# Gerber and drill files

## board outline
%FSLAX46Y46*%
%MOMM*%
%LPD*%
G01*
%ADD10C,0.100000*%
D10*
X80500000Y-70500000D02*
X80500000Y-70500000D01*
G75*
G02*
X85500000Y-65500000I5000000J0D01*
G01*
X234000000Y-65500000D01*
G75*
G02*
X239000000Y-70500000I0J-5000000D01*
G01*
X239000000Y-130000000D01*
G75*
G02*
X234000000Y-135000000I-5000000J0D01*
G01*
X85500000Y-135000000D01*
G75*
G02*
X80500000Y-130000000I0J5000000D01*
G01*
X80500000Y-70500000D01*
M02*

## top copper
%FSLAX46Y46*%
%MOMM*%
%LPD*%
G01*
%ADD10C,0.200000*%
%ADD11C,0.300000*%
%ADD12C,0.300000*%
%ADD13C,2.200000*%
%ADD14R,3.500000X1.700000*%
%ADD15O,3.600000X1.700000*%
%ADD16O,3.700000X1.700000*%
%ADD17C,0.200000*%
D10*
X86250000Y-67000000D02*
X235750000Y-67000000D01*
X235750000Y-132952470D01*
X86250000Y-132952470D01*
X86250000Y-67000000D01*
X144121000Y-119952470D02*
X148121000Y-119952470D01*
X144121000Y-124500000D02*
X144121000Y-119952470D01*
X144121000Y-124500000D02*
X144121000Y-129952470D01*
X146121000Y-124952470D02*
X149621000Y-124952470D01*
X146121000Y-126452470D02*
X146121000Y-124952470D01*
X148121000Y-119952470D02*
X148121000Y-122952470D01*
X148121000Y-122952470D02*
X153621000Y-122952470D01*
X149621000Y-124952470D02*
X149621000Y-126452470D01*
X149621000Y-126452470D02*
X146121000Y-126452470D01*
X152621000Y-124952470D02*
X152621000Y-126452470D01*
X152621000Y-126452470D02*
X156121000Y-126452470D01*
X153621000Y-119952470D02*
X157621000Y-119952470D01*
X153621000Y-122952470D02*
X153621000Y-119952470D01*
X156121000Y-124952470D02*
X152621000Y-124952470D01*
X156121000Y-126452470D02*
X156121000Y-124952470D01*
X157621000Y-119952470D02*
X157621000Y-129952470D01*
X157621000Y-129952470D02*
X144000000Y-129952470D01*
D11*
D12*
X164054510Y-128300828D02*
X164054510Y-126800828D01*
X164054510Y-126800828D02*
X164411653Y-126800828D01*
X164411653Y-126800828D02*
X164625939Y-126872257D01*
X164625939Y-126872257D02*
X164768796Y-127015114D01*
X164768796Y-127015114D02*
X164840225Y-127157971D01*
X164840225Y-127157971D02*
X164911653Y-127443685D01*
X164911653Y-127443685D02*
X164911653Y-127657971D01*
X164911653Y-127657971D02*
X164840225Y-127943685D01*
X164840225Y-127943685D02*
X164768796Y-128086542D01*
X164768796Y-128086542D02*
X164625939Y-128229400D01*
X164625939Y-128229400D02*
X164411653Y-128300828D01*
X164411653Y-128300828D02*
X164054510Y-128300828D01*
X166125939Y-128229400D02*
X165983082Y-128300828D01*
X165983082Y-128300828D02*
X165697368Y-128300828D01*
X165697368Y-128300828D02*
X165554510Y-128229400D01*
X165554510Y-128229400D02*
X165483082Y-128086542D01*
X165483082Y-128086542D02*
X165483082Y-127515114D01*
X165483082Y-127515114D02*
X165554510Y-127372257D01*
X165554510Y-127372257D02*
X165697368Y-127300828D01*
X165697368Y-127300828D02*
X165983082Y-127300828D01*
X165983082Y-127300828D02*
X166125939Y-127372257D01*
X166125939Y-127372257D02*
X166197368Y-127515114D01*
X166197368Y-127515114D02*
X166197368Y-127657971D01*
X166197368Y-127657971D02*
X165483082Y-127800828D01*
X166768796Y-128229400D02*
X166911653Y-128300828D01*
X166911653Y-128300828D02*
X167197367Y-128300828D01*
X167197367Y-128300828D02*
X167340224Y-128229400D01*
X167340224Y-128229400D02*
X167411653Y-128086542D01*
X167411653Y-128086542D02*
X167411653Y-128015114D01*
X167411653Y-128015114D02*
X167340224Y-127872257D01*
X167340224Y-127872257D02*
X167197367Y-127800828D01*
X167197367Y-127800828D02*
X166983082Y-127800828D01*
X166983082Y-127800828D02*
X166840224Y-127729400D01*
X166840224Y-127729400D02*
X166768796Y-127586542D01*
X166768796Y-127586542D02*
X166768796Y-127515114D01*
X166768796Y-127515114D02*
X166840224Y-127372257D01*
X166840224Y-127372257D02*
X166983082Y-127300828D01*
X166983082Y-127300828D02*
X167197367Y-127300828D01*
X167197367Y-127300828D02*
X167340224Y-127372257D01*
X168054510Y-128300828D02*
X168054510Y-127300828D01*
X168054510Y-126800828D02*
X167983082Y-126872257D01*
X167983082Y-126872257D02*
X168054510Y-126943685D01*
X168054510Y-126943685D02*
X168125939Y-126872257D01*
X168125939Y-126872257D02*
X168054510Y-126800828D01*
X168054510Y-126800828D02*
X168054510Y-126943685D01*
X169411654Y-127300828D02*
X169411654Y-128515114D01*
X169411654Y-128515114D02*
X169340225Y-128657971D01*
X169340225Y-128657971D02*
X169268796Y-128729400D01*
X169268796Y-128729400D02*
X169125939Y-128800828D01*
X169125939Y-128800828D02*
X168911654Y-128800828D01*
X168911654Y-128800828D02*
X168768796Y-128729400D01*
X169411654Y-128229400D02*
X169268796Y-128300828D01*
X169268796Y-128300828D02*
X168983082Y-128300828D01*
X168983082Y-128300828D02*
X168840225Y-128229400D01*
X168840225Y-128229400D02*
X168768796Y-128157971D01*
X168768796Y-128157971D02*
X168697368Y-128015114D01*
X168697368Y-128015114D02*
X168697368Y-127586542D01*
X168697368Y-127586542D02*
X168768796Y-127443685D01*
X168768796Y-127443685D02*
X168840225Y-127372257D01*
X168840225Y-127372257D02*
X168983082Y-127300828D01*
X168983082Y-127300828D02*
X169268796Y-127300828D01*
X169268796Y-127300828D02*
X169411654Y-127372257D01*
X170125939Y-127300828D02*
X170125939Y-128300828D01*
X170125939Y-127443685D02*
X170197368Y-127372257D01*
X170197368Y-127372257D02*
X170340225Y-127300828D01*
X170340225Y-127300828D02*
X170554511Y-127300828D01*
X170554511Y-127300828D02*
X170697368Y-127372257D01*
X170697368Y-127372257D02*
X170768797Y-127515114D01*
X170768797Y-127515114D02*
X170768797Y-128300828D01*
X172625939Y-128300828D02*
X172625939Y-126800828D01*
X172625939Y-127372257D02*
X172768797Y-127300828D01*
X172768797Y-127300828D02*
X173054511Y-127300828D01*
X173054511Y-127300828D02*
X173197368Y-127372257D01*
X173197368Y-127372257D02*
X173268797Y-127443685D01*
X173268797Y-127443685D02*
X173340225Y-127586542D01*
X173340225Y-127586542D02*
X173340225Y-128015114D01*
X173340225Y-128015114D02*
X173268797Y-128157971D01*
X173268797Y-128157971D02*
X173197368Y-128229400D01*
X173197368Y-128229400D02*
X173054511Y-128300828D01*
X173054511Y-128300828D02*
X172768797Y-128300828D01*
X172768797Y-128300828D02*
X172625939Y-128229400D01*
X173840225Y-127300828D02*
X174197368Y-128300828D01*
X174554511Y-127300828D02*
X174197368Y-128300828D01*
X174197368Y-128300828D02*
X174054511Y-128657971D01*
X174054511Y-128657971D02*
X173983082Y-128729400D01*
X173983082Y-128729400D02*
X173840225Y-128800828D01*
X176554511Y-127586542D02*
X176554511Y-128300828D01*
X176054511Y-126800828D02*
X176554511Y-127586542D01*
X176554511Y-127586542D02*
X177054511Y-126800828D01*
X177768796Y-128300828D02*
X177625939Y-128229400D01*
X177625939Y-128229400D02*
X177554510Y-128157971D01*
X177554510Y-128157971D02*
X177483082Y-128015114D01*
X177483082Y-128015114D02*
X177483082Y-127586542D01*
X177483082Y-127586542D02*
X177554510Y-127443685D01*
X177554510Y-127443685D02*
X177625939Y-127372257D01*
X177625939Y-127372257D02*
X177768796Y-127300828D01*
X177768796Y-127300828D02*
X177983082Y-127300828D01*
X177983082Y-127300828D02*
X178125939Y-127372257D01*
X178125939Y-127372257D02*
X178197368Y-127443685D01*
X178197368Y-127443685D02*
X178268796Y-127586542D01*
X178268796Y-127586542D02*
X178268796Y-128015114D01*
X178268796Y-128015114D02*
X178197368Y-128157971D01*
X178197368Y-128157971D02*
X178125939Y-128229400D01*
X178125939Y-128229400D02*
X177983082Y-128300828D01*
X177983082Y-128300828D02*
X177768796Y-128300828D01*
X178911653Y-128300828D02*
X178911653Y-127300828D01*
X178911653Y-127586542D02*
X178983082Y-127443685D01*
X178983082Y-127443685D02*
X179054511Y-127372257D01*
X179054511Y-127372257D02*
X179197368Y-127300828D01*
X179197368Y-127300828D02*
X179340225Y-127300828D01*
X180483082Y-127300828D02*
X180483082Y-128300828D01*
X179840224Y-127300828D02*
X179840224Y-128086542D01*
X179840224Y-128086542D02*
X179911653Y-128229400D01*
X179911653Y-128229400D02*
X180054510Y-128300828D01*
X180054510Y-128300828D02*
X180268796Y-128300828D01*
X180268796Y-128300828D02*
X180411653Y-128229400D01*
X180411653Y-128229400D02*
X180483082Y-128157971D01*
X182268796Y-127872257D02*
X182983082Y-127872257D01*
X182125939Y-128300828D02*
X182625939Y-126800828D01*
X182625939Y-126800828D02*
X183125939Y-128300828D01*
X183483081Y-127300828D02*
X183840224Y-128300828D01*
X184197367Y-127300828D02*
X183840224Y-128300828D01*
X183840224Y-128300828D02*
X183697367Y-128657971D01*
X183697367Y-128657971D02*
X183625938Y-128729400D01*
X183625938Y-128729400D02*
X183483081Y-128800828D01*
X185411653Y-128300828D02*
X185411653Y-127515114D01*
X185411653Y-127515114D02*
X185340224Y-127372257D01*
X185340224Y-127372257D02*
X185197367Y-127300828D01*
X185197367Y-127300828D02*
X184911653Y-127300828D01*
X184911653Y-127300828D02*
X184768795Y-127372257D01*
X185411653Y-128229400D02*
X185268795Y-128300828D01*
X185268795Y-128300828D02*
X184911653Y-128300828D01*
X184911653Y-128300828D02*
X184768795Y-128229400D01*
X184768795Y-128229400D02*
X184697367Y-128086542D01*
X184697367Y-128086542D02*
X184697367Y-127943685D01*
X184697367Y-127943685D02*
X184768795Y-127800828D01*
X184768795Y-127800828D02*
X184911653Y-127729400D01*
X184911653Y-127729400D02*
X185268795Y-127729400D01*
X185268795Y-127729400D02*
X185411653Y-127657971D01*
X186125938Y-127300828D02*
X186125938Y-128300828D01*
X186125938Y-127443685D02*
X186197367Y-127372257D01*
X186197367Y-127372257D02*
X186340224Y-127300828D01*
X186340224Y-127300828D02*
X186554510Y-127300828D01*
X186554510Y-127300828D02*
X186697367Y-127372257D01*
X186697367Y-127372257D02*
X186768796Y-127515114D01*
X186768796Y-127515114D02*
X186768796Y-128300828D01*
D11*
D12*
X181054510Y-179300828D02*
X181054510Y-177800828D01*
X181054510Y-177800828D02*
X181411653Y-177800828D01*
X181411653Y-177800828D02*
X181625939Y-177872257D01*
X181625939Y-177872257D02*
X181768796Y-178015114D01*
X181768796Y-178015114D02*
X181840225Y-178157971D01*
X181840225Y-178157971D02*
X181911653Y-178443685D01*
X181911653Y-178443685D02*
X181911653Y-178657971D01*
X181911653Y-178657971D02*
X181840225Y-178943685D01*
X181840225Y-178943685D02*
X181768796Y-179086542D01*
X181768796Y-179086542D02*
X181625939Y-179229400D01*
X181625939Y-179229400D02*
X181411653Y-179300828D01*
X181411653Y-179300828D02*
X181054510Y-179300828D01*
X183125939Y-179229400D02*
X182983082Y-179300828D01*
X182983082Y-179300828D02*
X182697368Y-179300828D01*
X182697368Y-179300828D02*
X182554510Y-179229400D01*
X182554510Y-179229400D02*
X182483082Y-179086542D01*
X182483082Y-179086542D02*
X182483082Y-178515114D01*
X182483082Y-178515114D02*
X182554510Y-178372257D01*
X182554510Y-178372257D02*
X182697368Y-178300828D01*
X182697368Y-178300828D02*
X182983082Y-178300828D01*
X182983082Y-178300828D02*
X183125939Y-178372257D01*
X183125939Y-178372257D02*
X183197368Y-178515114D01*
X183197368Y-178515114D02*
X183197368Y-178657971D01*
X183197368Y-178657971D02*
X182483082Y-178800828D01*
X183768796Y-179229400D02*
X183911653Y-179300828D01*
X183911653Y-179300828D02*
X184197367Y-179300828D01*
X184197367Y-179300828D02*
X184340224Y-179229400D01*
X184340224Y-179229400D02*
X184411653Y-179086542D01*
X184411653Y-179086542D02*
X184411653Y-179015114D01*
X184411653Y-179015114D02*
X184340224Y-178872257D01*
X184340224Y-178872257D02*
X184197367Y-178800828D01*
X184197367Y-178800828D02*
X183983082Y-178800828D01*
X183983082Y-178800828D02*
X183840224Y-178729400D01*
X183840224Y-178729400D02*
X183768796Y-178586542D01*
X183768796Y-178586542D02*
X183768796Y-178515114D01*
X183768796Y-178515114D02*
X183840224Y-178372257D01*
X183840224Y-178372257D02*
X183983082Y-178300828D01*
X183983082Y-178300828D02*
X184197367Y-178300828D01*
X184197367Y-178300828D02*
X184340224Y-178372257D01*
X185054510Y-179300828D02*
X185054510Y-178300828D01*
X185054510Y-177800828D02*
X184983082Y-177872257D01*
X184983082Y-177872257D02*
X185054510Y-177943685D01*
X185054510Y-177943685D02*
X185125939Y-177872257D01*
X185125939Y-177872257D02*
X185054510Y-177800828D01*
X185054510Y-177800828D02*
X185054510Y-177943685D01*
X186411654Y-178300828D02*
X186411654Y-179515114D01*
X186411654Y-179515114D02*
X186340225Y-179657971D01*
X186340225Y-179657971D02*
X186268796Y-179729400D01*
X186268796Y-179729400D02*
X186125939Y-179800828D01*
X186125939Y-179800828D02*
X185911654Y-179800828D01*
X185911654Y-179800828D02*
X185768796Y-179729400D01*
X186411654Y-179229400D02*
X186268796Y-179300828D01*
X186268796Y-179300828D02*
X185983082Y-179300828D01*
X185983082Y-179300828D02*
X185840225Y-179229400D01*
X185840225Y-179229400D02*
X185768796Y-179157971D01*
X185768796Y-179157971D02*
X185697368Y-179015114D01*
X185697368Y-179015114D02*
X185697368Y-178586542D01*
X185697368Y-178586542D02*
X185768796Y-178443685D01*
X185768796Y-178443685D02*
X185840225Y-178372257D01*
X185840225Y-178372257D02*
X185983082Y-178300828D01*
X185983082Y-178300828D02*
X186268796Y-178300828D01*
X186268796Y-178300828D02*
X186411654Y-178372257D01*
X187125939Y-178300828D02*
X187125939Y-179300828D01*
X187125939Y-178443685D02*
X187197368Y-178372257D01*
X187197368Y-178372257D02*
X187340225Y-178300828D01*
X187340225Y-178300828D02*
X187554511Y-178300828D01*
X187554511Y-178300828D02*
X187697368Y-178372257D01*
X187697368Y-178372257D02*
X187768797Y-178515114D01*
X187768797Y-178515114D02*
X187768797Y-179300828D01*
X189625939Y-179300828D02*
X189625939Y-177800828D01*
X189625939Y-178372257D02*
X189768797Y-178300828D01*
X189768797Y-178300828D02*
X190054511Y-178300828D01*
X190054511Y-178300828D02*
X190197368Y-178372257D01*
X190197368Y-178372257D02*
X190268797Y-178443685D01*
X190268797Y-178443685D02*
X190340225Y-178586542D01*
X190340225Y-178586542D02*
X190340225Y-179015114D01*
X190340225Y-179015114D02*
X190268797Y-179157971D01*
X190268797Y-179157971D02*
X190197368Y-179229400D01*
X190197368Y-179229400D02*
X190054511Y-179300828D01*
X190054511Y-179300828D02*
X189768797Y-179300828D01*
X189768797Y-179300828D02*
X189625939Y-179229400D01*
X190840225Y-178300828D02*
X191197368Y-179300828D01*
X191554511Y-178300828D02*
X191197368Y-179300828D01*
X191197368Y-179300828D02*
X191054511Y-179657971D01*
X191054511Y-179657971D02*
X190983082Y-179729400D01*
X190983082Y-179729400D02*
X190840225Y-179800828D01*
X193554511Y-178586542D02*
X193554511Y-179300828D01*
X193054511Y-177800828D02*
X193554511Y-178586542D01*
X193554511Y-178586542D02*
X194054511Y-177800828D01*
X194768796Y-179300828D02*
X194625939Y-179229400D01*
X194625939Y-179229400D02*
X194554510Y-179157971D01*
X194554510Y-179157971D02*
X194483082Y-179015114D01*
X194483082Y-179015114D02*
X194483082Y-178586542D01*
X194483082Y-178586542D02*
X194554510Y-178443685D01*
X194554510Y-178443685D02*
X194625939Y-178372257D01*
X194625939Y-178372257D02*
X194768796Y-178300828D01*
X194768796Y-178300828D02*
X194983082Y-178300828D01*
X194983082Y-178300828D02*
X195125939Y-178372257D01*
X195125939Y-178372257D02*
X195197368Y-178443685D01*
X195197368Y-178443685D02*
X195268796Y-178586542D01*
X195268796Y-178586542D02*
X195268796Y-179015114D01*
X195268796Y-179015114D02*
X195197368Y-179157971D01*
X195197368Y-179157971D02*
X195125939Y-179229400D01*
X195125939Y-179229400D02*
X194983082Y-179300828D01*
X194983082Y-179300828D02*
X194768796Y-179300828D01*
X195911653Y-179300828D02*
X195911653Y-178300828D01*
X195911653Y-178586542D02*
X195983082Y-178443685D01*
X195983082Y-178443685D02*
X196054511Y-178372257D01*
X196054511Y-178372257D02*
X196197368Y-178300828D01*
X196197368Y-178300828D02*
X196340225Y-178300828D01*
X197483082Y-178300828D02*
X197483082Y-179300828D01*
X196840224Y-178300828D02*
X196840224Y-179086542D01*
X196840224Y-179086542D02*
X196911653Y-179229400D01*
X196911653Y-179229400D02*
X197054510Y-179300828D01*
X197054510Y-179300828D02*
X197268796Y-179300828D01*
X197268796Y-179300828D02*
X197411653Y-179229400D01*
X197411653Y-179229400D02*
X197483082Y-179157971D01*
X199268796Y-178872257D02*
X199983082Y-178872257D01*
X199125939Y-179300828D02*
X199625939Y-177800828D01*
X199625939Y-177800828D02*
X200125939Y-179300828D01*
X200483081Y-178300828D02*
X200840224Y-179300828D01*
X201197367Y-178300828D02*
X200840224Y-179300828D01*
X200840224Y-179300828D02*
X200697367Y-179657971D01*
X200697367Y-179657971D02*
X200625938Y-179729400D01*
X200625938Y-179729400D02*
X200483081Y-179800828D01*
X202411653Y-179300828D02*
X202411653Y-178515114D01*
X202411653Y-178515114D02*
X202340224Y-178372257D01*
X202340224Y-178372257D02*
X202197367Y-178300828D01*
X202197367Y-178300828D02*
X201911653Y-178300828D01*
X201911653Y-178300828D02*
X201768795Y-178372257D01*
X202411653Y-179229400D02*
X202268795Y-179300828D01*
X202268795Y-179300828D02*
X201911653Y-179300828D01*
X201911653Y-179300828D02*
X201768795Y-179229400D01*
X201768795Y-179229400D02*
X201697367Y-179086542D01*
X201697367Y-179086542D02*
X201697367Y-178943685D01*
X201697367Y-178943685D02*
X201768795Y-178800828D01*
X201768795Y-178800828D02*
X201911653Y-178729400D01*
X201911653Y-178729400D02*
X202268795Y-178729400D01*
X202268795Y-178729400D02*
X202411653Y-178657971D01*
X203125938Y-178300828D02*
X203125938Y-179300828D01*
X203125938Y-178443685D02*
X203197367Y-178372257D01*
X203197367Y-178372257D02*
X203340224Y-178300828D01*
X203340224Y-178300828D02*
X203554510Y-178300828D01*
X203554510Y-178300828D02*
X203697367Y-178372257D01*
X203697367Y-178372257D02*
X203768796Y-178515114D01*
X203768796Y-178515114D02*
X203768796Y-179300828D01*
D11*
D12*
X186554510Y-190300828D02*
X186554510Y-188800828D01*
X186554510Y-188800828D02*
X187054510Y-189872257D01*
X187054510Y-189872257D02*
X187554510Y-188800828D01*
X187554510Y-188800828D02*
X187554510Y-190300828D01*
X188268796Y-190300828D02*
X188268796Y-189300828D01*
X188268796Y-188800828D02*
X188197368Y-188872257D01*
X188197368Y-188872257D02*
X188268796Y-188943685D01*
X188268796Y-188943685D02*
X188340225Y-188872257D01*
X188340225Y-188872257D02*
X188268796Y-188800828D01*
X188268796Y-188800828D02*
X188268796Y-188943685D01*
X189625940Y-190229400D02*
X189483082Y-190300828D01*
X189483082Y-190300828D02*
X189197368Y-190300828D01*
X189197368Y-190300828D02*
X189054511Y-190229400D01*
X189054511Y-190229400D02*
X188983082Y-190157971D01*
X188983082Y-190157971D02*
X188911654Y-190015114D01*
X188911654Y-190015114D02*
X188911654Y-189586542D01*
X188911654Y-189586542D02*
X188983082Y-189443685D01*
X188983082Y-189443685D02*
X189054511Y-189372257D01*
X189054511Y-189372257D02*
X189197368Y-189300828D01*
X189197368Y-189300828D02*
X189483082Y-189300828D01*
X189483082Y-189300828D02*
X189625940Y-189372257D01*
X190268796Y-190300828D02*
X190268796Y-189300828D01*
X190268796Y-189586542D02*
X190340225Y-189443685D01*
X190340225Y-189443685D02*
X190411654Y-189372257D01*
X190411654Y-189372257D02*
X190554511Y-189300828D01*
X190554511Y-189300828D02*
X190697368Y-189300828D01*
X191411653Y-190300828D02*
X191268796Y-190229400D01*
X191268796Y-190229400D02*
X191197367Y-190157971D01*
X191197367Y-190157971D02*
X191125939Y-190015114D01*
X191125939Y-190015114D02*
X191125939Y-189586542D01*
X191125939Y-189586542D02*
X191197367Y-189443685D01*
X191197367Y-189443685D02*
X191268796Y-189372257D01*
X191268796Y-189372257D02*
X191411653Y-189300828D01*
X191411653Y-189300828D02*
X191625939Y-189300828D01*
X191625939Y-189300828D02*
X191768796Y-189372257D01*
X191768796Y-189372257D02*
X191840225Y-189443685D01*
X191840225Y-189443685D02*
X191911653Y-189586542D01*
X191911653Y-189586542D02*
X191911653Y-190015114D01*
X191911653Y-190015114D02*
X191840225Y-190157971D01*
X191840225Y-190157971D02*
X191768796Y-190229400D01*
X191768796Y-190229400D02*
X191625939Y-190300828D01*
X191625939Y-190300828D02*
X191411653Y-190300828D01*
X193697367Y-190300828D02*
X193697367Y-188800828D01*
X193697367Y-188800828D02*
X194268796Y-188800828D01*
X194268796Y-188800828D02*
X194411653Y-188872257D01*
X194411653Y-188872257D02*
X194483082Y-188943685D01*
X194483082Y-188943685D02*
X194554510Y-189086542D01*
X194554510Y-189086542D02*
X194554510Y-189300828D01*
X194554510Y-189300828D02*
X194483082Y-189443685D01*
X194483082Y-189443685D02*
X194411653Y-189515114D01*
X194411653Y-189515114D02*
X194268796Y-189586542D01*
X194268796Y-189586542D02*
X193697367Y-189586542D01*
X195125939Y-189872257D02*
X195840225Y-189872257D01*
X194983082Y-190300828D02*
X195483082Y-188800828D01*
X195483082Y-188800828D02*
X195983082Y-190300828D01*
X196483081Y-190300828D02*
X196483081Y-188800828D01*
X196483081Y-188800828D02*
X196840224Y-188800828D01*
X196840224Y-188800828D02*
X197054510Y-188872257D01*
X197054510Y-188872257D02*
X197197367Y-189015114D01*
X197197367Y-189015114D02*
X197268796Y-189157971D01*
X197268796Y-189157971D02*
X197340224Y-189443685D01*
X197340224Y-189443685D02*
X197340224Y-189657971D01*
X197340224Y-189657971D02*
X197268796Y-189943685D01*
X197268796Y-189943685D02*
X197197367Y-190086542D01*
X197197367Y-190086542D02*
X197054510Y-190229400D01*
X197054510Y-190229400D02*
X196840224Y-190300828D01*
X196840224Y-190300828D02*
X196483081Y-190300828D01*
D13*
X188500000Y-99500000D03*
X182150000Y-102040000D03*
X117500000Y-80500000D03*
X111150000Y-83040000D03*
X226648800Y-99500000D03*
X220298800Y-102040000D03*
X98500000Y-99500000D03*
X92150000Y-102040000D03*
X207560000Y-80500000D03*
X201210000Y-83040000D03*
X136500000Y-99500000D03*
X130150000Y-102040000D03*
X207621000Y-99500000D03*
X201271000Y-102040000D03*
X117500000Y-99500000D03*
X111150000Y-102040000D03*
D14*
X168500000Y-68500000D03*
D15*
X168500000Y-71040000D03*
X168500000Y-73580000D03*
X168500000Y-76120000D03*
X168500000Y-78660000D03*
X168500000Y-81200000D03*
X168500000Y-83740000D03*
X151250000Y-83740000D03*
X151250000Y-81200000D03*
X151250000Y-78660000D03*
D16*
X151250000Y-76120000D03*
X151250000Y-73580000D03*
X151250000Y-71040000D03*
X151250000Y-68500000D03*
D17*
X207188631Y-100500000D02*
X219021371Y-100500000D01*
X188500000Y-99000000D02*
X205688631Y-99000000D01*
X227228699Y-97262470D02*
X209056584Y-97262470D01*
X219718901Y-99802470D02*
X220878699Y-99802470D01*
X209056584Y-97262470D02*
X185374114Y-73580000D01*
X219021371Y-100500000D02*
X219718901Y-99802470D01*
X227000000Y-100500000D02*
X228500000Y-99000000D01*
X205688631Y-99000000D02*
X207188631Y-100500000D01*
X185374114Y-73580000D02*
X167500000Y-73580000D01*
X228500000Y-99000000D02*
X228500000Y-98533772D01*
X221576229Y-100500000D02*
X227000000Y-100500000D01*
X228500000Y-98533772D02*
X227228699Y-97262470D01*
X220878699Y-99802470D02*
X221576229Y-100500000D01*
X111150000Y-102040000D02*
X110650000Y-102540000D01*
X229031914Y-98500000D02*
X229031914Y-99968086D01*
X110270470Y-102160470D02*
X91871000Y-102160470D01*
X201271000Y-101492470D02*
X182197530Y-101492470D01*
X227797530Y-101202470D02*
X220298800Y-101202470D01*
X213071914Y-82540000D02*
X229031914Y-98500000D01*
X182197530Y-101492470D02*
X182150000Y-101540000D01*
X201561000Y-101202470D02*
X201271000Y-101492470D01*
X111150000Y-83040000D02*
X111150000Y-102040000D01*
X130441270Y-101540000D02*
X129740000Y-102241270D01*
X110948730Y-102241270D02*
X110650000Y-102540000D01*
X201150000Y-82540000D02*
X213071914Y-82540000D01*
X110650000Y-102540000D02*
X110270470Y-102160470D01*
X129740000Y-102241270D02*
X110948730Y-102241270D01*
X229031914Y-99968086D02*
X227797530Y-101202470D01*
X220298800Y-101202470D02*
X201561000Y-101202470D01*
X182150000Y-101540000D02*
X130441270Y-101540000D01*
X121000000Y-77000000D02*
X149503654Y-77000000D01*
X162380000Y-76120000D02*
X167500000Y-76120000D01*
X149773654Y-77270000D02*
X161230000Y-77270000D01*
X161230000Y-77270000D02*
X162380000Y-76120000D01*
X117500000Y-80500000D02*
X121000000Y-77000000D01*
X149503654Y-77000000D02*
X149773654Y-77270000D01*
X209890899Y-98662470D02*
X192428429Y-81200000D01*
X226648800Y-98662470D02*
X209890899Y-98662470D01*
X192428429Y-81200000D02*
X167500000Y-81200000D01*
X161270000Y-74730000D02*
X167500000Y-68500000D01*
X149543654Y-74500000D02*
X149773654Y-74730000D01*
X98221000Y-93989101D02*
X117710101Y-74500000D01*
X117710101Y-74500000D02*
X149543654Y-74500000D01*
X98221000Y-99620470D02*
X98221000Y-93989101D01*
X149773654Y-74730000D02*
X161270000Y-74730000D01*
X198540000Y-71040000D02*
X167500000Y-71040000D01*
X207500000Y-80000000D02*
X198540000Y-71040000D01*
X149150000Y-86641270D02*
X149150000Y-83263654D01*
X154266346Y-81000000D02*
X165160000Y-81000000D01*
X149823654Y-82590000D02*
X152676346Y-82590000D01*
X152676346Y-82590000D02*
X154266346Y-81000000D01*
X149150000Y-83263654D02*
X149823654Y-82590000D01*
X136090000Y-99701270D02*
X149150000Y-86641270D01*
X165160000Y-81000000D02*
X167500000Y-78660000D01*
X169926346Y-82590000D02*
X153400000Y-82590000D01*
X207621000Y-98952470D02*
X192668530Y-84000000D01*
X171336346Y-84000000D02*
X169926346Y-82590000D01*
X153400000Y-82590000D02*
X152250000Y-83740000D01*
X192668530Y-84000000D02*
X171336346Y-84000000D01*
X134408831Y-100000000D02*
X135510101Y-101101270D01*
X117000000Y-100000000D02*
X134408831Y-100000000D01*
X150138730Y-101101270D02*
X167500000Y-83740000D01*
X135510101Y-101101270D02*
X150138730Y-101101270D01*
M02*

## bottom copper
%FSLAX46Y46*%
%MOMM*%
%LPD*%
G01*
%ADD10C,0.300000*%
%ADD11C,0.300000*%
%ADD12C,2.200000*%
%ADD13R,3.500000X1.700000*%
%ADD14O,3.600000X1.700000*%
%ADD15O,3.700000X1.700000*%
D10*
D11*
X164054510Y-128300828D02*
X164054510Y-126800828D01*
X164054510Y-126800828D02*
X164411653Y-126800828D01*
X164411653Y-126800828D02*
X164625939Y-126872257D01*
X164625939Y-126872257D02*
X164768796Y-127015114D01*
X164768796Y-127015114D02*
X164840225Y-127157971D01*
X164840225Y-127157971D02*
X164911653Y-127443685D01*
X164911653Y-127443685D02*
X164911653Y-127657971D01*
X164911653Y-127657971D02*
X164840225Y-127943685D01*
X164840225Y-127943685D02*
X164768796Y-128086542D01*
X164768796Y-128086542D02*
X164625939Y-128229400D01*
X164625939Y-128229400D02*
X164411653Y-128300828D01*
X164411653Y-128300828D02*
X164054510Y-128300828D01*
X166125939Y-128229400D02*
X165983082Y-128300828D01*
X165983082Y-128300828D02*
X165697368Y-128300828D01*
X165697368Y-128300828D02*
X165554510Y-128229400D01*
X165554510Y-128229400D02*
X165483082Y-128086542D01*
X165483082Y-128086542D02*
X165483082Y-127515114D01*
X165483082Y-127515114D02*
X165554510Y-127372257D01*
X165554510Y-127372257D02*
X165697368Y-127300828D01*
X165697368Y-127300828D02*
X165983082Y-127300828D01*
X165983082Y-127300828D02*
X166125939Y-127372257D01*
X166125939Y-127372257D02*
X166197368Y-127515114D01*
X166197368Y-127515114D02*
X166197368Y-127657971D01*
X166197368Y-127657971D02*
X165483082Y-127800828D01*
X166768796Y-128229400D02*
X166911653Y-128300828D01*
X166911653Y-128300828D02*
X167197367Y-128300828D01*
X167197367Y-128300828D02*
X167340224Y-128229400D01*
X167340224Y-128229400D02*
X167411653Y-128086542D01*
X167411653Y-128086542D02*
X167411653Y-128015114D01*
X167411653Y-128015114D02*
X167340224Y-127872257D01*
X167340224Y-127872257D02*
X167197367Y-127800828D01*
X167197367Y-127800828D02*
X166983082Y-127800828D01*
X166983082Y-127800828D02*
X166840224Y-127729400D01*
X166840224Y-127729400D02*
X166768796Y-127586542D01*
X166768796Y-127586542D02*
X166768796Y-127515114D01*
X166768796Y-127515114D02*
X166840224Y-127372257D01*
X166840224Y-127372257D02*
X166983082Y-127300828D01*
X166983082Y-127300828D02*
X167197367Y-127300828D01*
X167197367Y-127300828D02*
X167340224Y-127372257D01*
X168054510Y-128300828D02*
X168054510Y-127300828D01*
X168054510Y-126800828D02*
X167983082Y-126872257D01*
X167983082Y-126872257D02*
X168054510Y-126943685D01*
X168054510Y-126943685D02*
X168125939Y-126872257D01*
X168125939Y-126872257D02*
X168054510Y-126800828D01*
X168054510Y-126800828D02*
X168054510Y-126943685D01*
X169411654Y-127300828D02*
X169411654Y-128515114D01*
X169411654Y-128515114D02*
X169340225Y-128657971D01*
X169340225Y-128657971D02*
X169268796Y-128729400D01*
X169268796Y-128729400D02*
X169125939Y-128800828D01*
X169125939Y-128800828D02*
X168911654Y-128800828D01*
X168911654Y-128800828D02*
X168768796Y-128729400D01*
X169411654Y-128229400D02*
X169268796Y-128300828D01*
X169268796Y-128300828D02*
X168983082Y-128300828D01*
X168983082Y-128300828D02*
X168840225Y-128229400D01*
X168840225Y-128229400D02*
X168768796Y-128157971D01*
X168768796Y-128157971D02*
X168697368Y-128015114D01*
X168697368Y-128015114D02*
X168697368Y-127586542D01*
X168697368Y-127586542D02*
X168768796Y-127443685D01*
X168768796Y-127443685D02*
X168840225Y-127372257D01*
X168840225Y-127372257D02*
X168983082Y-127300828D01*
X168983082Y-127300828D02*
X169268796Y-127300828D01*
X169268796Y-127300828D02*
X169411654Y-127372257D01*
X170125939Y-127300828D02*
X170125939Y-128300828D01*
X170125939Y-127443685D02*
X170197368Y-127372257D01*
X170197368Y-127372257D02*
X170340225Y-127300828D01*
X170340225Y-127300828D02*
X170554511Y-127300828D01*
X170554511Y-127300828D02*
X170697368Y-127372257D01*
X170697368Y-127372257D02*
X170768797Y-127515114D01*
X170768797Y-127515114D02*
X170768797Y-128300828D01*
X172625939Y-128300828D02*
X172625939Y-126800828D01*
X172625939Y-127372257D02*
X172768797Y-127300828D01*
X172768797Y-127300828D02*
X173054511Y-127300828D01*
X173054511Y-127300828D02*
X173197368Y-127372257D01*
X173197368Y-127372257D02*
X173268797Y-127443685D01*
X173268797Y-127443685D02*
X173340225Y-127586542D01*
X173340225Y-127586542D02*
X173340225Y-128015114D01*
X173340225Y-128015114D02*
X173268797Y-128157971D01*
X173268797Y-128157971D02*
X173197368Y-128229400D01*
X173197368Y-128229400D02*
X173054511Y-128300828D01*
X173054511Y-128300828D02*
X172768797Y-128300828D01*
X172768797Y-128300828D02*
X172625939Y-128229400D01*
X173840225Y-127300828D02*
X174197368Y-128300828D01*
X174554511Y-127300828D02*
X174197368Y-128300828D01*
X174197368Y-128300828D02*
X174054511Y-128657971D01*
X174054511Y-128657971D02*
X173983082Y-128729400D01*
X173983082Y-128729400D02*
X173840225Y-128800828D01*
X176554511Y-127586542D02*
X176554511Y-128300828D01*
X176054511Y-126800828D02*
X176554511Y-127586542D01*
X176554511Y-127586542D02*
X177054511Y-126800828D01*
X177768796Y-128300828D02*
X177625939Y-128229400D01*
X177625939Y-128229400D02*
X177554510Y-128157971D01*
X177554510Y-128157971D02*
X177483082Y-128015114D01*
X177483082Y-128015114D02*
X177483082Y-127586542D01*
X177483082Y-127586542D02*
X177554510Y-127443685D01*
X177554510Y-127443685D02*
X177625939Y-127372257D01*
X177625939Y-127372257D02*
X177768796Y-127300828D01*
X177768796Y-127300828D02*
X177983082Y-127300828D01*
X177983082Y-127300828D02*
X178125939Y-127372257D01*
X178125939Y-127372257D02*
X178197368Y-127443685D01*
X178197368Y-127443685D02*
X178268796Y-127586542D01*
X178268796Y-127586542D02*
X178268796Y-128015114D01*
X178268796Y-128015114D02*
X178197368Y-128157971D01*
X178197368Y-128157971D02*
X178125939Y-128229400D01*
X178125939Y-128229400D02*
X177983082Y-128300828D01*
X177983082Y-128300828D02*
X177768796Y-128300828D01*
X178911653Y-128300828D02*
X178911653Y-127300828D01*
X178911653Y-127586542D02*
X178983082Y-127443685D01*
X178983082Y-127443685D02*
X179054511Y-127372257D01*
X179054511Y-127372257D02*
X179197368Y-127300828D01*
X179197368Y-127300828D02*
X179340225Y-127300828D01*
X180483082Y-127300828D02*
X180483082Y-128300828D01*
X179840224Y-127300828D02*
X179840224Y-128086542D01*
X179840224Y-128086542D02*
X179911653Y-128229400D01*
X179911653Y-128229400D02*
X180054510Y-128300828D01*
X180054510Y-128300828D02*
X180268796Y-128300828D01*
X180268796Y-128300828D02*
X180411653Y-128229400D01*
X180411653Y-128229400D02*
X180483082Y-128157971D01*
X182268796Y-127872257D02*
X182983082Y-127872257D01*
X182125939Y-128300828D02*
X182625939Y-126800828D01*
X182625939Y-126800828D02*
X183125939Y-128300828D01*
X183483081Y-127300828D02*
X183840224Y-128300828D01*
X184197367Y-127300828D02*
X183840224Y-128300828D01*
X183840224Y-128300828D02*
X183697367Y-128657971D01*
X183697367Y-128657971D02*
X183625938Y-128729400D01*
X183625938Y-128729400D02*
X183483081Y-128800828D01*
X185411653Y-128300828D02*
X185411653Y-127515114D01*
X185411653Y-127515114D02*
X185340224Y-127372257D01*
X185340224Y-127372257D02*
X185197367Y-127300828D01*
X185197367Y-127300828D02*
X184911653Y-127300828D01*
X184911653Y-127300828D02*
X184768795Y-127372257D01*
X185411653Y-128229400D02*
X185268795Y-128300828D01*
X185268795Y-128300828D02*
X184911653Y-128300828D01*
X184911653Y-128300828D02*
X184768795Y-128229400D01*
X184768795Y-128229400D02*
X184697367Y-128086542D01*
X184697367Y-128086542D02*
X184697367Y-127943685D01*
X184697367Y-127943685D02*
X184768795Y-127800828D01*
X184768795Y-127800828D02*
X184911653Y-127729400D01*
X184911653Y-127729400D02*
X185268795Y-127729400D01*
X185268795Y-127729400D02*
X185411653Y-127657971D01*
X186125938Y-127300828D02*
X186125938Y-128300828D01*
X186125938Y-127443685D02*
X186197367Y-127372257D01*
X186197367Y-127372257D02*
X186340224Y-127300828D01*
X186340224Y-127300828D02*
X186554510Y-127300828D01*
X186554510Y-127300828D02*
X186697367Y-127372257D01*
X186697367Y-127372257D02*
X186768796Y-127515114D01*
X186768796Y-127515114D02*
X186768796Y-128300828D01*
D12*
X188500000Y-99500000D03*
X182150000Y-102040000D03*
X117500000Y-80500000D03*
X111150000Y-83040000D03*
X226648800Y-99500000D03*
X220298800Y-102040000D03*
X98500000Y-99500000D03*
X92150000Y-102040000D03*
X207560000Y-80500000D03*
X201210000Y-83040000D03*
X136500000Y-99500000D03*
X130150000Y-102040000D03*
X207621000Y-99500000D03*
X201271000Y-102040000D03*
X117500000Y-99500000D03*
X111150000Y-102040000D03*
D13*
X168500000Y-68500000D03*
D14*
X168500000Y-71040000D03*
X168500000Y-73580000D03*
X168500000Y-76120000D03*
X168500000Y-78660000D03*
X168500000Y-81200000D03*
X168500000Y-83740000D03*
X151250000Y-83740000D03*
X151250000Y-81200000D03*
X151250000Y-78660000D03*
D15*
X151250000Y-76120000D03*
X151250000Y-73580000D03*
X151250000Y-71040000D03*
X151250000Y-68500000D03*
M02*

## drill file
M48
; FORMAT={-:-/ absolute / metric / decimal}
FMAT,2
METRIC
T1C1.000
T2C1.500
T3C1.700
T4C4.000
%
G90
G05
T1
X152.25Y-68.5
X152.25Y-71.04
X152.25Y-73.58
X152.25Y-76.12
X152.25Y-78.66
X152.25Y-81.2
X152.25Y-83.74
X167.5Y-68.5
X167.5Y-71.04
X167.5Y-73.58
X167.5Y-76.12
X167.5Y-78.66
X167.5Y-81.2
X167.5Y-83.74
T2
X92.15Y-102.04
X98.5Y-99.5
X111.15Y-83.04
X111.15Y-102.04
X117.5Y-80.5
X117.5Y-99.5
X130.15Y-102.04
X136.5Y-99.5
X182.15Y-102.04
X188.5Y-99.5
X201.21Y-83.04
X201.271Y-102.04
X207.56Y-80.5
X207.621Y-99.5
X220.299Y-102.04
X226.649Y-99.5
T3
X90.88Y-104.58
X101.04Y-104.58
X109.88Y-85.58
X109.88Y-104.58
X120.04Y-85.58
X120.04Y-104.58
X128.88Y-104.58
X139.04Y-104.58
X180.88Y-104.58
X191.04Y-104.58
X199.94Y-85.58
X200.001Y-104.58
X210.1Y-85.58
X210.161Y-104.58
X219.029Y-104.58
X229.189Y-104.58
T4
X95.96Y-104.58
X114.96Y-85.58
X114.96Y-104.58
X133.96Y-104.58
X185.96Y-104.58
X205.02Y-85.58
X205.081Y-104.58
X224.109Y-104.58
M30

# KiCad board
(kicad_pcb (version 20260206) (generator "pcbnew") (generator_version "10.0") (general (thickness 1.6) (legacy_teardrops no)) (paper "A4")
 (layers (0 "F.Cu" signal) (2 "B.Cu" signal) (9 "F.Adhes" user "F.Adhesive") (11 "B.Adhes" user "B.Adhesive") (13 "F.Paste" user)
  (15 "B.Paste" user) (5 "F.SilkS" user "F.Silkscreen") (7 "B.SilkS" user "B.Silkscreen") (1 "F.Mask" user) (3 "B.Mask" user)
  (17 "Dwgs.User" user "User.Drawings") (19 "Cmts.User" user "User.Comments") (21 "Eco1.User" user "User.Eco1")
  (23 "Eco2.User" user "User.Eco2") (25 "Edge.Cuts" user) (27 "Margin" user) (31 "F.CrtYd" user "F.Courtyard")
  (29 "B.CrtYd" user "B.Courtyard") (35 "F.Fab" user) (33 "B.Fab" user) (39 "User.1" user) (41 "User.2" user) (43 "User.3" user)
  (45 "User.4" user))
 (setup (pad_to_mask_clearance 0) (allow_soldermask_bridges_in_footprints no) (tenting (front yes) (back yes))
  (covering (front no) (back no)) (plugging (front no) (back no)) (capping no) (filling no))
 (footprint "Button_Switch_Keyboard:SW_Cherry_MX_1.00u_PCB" (layer "F.Cu") (at 188.5 99.5)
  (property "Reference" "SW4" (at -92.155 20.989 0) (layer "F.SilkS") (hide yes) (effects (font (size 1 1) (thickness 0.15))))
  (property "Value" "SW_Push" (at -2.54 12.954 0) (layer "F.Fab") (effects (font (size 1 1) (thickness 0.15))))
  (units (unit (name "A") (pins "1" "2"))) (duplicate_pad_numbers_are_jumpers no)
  (pad "" np_thru_hole circle (at -7.62 5.08) (size 1.7 1.7) (drill 1.7) (layers "*.Cu" "*.Mask"))
  (pad "" np_thru_hole circle (at -2.54 5.08) (size 4 4) (drill 4) (layers "*.Cu" "*.Mask"))
  (pad "" np_thru_hole circle (at 2.54 5.08) (size 1.7 1.7) (drill 1.7) (layers "*.Cu" "*.Mask"))
  (pad "1" thru_hole circle (at 0 0) (size 2.2 2.2) (drill 1.5) (layers "*.Cu" "*.Mask") (remove_unused_layers no)
   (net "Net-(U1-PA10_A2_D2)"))
  (pad "2" thru_hole circle (at -6.35 2.54) (size 2.2 2.2) (drill 1.5) (layers "*.Cu" "*.Mask") (remove_unused_layers no) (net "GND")))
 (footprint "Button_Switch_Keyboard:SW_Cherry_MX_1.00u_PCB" (layer "F.Cu") (at 117.5 80.5)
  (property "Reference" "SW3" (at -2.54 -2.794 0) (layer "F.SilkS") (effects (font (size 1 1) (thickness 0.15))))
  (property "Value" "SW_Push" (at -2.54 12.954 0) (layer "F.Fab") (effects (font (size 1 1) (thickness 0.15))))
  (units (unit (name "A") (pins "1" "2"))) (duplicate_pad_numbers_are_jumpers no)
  (pad "" np_thru_hole circle (at -7.62 5.08) (size 1.7 1.7) (drill 1.7) (layers "*.Cu" "*.Mask"))
  (pad "" np_thru_hole circle (at -2.54 5.08) (size 4 4) (drill 4) (layers "*.Cu" "*.Mask"))
  (pad "" np_thru_hole circle (at 2.54 5.08) (size 1.7 1.7) (drill 1.7) (layers "*.Cu" "*.Mask"))
  (pad "1" thru_hole circle (at 0 0) (size 2.2 2.2) (drill 1.5) (layers "*.Cu" "*.Mask") (remove_unused_layers no)
   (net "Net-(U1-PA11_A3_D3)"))
  (pad "2" thru_hole circle (at -6.35 2.54) (size 2.2 2.2) (drill 1.5) (layers "*.Cu" "*.Mask") (remove_unused_layers no) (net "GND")))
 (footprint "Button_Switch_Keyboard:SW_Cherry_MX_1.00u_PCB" (layer "F.Cu") (at 226.6488 99.5)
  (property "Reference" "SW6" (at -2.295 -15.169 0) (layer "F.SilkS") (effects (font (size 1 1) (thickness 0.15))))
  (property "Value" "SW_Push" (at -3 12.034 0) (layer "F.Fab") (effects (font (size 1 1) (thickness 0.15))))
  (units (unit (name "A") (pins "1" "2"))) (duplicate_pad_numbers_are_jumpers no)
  (pad "" np_thru_hole circle (at -7.62 5.08) (size 1.7 1.7) (drill 1.7) (layers "*.Cu" "*.Mask"))
  (pad "" np_thru_hole circle (at -2.54 5.08) (size 4 4) (drill 4) (layers "*.Cu" "*.Mask"))
  (pad "" np_thru_hole circle (at 2.54 5.08) (size 1.7 1.7) (drill 1.7) (layers "*.Cu" "*.Mask"))
  (pad "1" thru_hole circle (at 0 0) (size 2.2 2.2) (drill 1.5) (layers "*.Cu" "*.Mask") (remove_unused_layers no)
   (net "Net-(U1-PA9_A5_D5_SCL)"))
  (pad "2" thru_hole circle (at -6.35 2.54) (size 2.2 2.2) (drill 1.5) (layers "*.Cu" "*.Mask") (remove_unused_layers no) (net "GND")))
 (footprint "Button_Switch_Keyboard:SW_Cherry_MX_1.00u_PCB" (layer "F.Cu") (at 98.5 99.5)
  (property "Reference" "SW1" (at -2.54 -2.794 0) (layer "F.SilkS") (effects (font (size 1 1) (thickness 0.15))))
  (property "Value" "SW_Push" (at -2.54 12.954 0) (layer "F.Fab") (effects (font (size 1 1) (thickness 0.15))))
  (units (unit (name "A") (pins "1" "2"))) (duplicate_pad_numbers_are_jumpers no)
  (pad "" np_thru_hole circle (at -7.62 5.08) (size 1.7 1.7) (drill 1.7) (layers "*.Cu" "*.Mask"))
  (pad "" np_thru_hole circle (at -2.54 5.08) (size 4 4) (drill 4) (layers "*.Cu" "*.Mask"))
  (pad "" np_thru_hole circle (at 2.54 5.08) (size 1.7 1.7) (drill 1.7) (layers "*.Cu" "*.Mask"))
  (pad "1" thru_hole circle (at 0 0) (size 2.2 2.2) (drill 1.5) (layers "*.Cu" "*.Mask") (remove_unused_layers no)
   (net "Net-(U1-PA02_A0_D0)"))
  (pad "2" thru_hole circle (at -6.35 2.54) (size 2.2 2.2) (drill 1.5) (layers "*.Cu" "*.Mask") (remove_unused_layers no) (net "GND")))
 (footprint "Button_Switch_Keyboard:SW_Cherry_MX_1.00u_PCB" (layer "F.Cu") (at 207.56 80.5)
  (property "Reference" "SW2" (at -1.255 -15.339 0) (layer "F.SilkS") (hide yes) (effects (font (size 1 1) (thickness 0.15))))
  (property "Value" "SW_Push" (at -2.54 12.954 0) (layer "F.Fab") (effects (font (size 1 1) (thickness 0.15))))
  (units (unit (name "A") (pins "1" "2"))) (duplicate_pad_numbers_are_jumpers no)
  (pad "" np_thru_hole circle (at -7.62 5.08) (size 1.7 1.7) (drill 1.7) (layers "*.Cu" "*.Mask"))
  (pad "" np_thru_hole circle (at -2.54 5.08) (size 4 4) (drill 4) (layers "*.Cu" "*.Mask"))
  (pad "" np_thru_hole circle (at 2.54 5.08) (size 1.7 1.7) (drill 1.7) (layers "*.Cu" "*.Mask"))
  (pad "1" thru_hole circle (at 0 0) (size 2.2 2.2) (drill 1.5) (layers "*.Cu" "*.Mask") (remove_unused_layers no)
   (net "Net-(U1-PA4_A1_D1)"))
  (pad "2" thru_hole circle (at -6.35 2.54) (size 2.2 2.2) (drill 1.5) (layers "*.Cu" "*.Mask") (remove_unused_layers no) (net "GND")))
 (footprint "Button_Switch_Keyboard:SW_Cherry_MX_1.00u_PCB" (layer "F.Cu") (at 136.5 99.5)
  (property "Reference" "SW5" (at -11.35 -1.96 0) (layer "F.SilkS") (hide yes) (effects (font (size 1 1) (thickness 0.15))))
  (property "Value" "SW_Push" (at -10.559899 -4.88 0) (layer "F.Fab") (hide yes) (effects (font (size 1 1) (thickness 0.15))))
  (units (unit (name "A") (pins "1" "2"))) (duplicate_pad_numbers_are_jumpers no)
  (pad "" np_thru_hole circle (at -7.62 5.08) (size 1.7 1.7) (drill 1.7) (layers "*.Cu" "*.Mask"))
  (pad "" np_thru_hole circle (at -2.54 5.08) (size 4 4) (drill 4) (layers "*.Cu" "*.Mask"))
  (pad "" np_thru_hole circle (at 2.54 5.08) (size 1.7 1.7) (drill 1.7) (layers "*.Cu" "*.Mask"))
  (pad "1" thru_hole circle (at 0 0) (size 2.2 2.2) (drill 1.5) (layers "*.Cu" "*.Mask") (remove_unused_layers no)
   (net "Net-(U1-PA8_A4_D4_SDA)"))
  (pad "2" thru_hole circle (at -6.35 2.54) (size 2.2 2.2) (drill 1.5) (layers "*.Cu" "*.Mask") (remove_unused_layers no) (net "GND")))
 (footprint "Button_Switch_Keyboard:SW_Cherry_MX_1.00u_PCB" (layer "F.Cu") (at 207.621 99.5)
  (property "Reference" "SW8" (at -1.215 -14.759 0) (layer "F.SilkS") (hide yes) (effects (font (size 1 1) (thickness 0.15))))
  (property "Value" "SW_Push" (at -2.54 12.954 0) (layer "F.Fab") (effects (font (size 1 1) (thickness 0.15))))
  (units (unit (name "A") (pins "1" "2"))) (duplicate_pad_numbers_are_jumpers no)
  (pad "" np_thru_hole circle (at -7.62 5.08) (size 1.7 1.7) (drill 1.7) (layers "*.Cu" "*.Mask"))
  (pad "" np_thru_hole circle (at -2.54 5.08) (size 4 4) (drill 4) (layers "*.Cu" "*.Mask"))
  (pad "" np_thru_hole circle (at 2.54 5.08) (size 1.7 1.7) (drill 1.7) (layers "*.Cu" "*.Mask"))
  (pad "1" thru_hole circle (at 0 0) (size 2.2 2.2) (drill 1.5) (layers "*.Cu" "*.Mask") (remove_unused_layers no)
   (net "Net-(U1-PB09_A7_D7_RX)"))
  (pad "2" thru_hole circle (at -6.35 2.54) (size 2.2 2.2) (drill 1.5) (layers "*.Cu" "*.Mask") (remove_unused_layers no) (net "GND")))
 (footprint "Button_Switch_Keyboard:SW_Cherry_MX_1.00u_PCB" (layer "F.Cu") (at 117.5 99.5)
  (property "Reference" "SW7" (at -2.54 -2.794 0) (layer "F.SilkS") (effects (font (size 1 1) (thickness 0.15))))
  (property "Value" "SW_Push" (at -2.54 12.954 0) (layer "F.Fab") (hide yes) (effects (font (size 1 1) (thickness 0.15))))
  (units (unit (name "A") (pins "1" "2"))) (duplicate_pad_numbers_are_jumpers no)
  (pad "" np_thru_hole circle (at -7.62 5.08) (size 1.7 1.7) (drill 1.7) (layers "*.Cu" "*.Mask"))
  (pad "" np_thru_hole circle (at -2.54 5.08) (size 4 4) (drill 4) (layers "*.Cu" "*.Mask"))
  (pad "" np_thru_hole circle (at 2.54 5.08) (size 1.7 1.7) (drill 1.7) (layers "*.Cu" "*.Mask"))
  (pad "1" thru_hole circle (at 0 0) (size 2.2 2.2) (drill 1.5) (layers "*.Cu" "*.Mask") (remove_unused_layers no)
   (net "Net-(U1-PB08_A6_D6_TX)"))
  (pad "2" thru_hole circle (at -6.35 2.54) (size 2.2 2.2) (drill 1.5) (layers "*.Cu" "*.Mask") (remove_unused_layers no) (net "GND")))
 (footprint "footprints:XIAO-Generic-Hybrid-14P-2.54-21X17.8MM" (layer "B.Cu") (at 159.875 76.12 180)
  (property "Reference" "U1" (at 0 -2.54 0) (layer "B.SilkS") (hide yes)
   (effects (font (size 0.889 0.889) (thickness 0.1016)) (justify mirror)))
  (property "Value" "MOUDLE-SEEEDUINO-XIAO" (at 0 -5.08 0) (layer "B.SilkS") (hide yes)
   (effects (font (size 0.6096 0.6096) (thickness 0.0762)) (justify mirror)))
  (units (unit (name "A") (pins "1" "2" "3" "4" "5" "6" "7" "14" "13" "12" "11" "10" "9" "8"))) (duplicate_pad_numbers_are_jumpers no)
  (pad "1" thru_hole rect (at -7.625 7.62 180) (size 3.5 1.7) (drill 1 (offset -1 0)) (layers "*.Cu" "*.Mask") (remove_unused_layers no)
   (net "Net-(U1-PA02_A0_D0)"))
  (pad "2" thru_hole oval (at -7.625 5.08 180) (size 3.6 1.7) (drill 1 (offset -1 0)) (layers "*.Cu" "*.Mask") (remove_unused_layers no)
   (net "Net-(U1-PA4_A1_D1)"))
  (pad "3" thru_hole oval (at -7.625 2.54 180) (size 3.6 1.7) (drill 1 (offset -1 0)) (layers "*.Cu" "*.Mask") (remove_unused_layers no)
   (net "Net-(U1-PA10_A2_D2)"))
  (pad "4" thru_hole oval (at -7.625 0 180) (size 3.6 1.7) (drill 1 (offset -1 0)) (layers "*.Cu" "*.Mask") (remove_unused_layers no)
   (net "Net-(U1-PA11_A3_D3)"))
  (pad "5" thru_hole oval (at -7.625 -2.54 180) (size 3.6 1.7) (drill 1 (offset -1 0)) (layers "*.Cu" "*.Mask") (remove_unused_layers no)
   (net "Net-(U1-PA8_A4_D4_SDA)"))
  (pad "6" thru_hole oval (at -7.625 -5.08) (size 3.6 1.7) (drill 1 (offset 1 0)) (layers "*.Cu" "*.Mask") (remove_unused_layers no)
   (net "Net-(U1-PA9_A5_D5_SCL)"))
  (pad "7" thru_hole oval (at -7.625 -7.62 180) (size 3.6 1.7) (drill 1 (offset -1 0)) (layers "*.Cu" "*.Mask") (remove_unused_layers no)
   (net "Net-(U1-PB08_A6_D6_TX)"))
  (pad "8" thru_hole oval (at 7.625 -7.62 180) (size 3.6 1.7) (drill 1 (offset 1 0)) (layers "*.Cu" "*.Mask") (remove_unused_layers no)
   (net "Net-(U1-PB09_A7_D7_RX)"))
  (pad "9" thru_hole oval (at 7.625 -5.08 180) (size 3.6 1.7) (drill 1 (offset 1 0)) (layers "*.Cu" "*.Mask") (remove_unused_layers no)
   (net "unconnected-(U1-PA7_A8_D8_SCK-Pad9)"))
  (pad "10" thru_hole oval (at 7.625 -2.54 180) (size 3.6 1.7) (drill 1 (offset 1 0)) (layers "*.Cu" "*.Mask") (remove_unused_layers no)
   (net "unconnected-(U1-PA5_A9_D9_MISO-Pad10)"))
  (pad "11" thru_hole oval (at 7.625 0 180) (size 3.7 1.7) (drill 1 (offset 1 0)) (layers "*.Cu" "*.Mask") (remove_unused_layers no)
   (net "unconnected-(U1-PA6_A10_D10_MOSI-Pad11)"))
  (pad "12" thru_hole oval (at 7.625 2.54 180) (size 3.7 1.7) (drill 1 (offset 1 0)) (layers "*.Cu" "*.Mask") (remove_unused_layers no)
   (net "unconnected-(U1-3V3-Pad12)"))
  (pad "13" thru_hole oval (at 7.625 5.08 180) (size 3.7 1.7) (drill 1 (offset 1 0)) (layers "*.Cu" "*.Mask") (remove_unused_layers no)
   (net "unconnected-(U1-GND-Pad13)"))
  (pad "14" thru_hole oval (at 7.625 7.62 180) (size 3.7 1.7) (drill 1 (offset 1 0)) (layers "*.Cu" "*.Mask") (remove_unused_layers no)
   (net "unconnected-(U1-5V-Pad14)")))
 (gr_rect (start 86.25 67) (end 235.75 132.95247) (stroke (width 0.2) (type default)) (fill no) (layer "F.Cu"))
 (gr_line (start 144.121 119.95247) (end 148.121 119.95247) (stroke (width 0.2) (type default)) (layer "F.Cu"))
 (gr_line (start 144.121 124.5) (end 144.121 119.95247) (stroke (width 0.2) (type default)) (layer "F.Cu"))
 (gr_line (start 144.121 124.5) (end 144.121 129.95247) (stroke (width 0.2) (type default)) (layer "F.Cu"))
 (gr_line (start 146.121 124.95247) (end 149.621 124.95247) (stroke (width 0.2) (type default)) (layer "F.Cu"))
 (gr_line (start 146.121 126.45247) (end 146.121 124.95247) (stroke (width 0.2) (type default)) (layer "F.Cu"))
 (gr_line (start 148.121 119.95247) (end 148.121 122.95247) (stroke (width 0.2) (type default)) (layer "F.Cu"))
 (gr_line (start 148.121 122.95247) (end 153.621 122.95247) (stroke (width 0.2) (type default)) (layer "F.Cu"))
 (gr_line (start 149.621 124.95247) (end 149.621 126.45247) (stroke (width 0.2) (type default)) (layer "F.Cu"))
 (gr_line (start 149.621 126.45247) (end 146.121 126.45247) (stroke (width 0.2) (type default)) (layer "F.Cu"))
 (gr_line (start 152.621 124.95247) (end 152.621 126.45247) (stroke (width 0.2) (type default)) (layer "F.Cu"))
 (gr_line (start 152.621 126.45247) (end 156.121 126.45247) (stroke (width 0.2) (type default)) (layer "F.Cu"))
 (gr_line (start 153.621 119.95247) (end 157.621 119.95247) (stroke (width 0.2) (type default)) (layer "F.Cu"))
 (gr_line (start 153.621 122.95247) (end 153.621 119.95247) (stroke (width 0.2) (type default)) (layer "F.Cu"))
 (gr_line (start 156.121 124.95247) (end 152.621 124.95247) (stroke (width 0.2) (type default)) (layer "F.Cu"))
 (gr_line (start 156.121 126.45247) (end 156.121 124.95247) (stroke (width 0.2) (type default)) (layer "F.Cu"))
 (gr_line (start 157.621 119.95247) (end 157.621 129.95247) (stroke (width 0.2) (type default)) (layer "F.Cu"))
 (gr_line (start 157.621 129.95247) (end 144 129.95247) (stroke (width 0.2) (type default)) (layer "F.Cu"))
 (gr_rect (start 80.5 65.5) (end 239 135) (radius 5) (stroke (width 0.1) (type default)) (fill no) (layer "Edge.Cuts"))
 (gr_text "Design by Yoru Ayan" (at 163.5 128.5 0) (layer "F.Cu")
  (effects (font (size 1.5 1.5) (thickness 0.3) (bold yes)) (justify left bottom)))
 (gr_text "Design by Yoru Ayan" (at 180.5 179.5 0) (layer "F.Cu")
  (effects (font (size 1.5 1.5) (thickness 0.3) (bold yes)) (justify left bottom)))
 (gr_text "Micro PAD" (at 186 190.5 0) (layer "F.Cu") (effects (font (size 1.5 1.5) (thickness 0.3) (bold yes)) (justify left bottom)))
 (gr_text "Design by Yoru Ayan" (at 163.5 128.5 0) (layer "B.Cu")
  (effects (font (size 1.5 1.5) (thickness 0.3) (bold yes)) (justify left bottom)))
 (segment (start 207.188631 100.5) (end 219.021371 100.5) (width 0.2) (layer "F.Cu") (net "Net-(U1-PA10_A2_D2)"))
 (segment (start 188.5 99) (end 205.688631 99) (width 0.2) (layer "F.Cu") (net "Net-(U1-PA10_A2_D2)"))
 (segment (start 227.228699 97.26247) (end 209.056584 97.26247) (width 0.2) (layer "F.Cu") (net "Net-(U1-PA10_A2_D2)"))
 (segment (start 219.718901 99.80247) (end 220.878699 99.80247) (width 0.2) (layer "F.Cu") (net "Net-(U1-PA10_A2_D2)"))
 (segment (start 209.056584 97.26247) (end 185.374114 73.58) (width 0.2) (layer "F.Cu") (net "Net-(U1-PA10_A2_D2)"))
 (segment (start 219.021371 100.5) (end 219.718901 99.80247) (width 0.2) (layer "F.Cu") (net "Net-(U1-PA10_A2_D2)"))
 (segment (start 227 100.5) (end 228.5 99) (width 0.2) (layer "F.Cu") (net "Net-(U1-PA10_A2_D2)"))
 (segment (start 205.688631 99) (end 207.188631 100.5) (width 0.2) (layer "F.Cu") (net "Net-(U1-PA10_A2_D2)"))
 (segment (start 185.374114 73.58) (end 167.5 73.58) (width 0.2) (layer "F.Cu") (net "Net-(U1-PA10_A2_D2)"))
 (segment (start 228.5 99) (end 228.5 98.533772) (width 0.2) (layer "F.Cu") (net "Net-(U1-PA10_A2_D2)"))
 (segment (start 221.576229 100.5) (end 227 100.5) (width 0.2) (layer "F.Cu") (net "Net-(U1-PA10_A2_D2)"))
 (segment (start 228.5 98.533772) (end 227.228699 97.26247) (width 0.2) (layer "F.Cu") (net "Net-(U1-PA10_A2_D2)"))
 (segment (start 220.878699 99.80247) (end 221.576229 100.5) (width 0.2) (layer "F.Cu") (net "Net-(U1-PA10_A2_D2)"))
 (segment (start 111.15 102.04) (end 110.65 102.54) (width 0.2) (layer "F.Cu") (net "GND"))
 (segment (start 229.031914 98.5) (end 229.031914 99.968086) (width 0.2) (layer "F.Cu") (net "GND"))
 (segment (start 110.27047 102.16047) (end 91.871 102.16047) (width 0.2) (layer "F.Cu") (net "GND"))
 (segment (start 201.271 101.49247) (end 182.19753 101.49247) (width 0.2) (layer "F.Cu") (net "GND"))
 (segment (start 227.79753 101.20247) (end 220.2988 101.20247) (width 0.2) (layer "F.Cu") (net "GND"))
 (segment (start 213.071914 82.54) (end 229.031914 98.5) (width 0.2) (layer "F.Cu") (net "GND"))
 (segment (start 182.19753 101.49247) (end 182.15 101.54) (width 0.2) (layer "F.Cu") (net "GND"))
 (segment (start 201.561 101.20247) (end 201.271 101.49247) (width 0.2) (layer "F.Cu") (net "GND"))
 (segment (start 111.15 83.04) (end 111.15 102.04) (width 0.2) (layer "F.Cu") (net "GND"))
 (segment (start 130.44127 101.54) (end 129.74 102.24127) (width 0.2) (layer "F.Cu") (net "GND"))
 (segment (start 110.94873 102.24127) (end 110.65 102.54) (width 0.2) (layer "F.Cu") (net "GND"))
 (segment (start 201.15 82.54) (end 213.071914 82.54) (width 0.2) (layer "F.Cu") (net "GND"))
 (segment (start 110.65 102.54) (end 110.27047 102.16047) (width 0.2) (layer "F.Cu") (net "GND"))
 (segment (start 129.74 102.24127) (end 110.94873 102.24127) (width 0.2) (layer "F.Cu") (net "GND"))
 (segment (start 229.031914 99.968086) (end 227.79753 101.20247) (width 0.2) (layer "F.Cu") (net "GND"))
 (segment (start 220.2988 101.20247) (end 201.561 101.20247) (width 0.2) (layer "F.Cu") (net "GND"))
 (segment (start 182.15 101.54) (end 130.44127 101.54) (width 0.2) (layer "F.Cu") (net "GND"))
 (segment (start 121 77) (end 149.503654 77) (width 0.2) (layer "F.Cu") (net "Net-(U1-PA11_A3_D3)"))
 (segment (start 162.38 76.12) (end 167.5 76.12) (width 0.2) (layer "F.Cu") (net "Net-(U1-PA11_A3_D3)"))
 (segment (start 149.773654 77.27) (end 161.23 77.27) (width 0.2) (layer "F.Cu") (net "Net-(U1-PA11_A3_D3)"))
 (segment (start 161.23 77.27) (end 162.38 76.12) (width 0.2) (layer "F.Cu") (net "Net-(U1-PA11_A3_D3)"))
 (segment (start 117.5 80.5) (end 121 77) (width 0.2) (layer "F.Cu") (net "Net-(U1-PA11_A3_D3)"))
 (segment (start 149.503654 77) (end 149.773654 77.27) (width 0.2) (layer "F.Cu") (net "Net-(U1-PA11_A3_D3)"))
 (segment (start 209.890899 98.66247) (end 192.428429 81.2) (width 0.2) (layer "F.Cu") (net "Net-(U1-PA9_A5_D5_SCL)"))
 (segment (start 226.6488 98.66247) (end 209.890899 98.66247) (width 0.2) (layer "F.Cu") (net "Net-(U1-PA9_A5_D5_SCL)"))
 (segment (start 192.428429 81.2) (end 167.5 81.2) (width 0.2) (layer "F.Cu") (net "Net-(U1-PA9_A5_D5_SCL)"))
 (segment (start 161.27 74.73) (end 167.5 68.5) (width 0.2) (layer "F.Cu") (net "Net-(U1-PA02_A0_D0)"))
 (segment (start 149.543654 74.5) (end 149.773654 74.73) (width 0.2) (layer "F.Cu") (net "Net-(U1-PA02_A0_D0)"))
 (segment (start 98.221 93.989101) (end 117.710101 74.5) (width 0.2) (layer "F.Cu") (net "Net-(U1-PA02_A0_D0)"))
 (segment (start 117.710101 74.5) (end 149.543654 74.5) (width 0.2) (layer "F.Cu") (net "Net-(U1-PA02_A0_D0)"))
 (segment (start 98.221 99.62047) (end 98.221 93.989101) (width 0.2) (layer "F.Cu") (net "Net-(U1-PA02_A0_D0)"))
 (segment (start 149.773654 74.73) (end 161.27 74.73) (width 0.2) (layer "F.Cu") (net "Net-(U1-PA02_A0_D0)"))
 (segment (start 198.54 71.04) (end 167.5 71.04) (width 0.2) (layer "F.Cu") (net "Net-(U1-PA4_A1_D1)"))
 (segment (start 207.5 80) (end 198.54 71.04) (width 0.2) (layer "F.Cu") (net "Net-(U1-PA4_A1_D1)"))
 (segment (start 149.15 86.64127) (end 149.15 83.263654) (width 0.2) (layer "F.Cu") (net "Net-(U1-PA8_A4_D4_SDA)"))
 (segment (start 154.266346 81) (end 165.16 81) (width 0.2) (layer "F.Cu") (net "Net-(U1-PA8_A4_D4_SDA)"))
 (segment (start 149.823654 82.59) (end 152.676346 82.59) (width 0.2) (layer "F.Cu") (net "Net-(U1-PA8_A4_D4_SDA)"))
 (segment (start 152.676346 82.59) (end 154.266346 81) (width 0.2) (layer "F.Cu") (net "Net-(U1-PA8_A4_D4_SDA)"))
 (segment (start 149.15 83.263654) (end 149.823654 82.59) (width 0.2) (layer "F.Cu") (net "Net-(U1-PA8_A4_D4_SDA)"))
 (segment (start 136.09 99.70127) (end 149.15 86.64127) (width 0.2) (layer "F.Cu") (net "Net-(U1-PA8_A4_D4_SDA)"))
 (segment (start 165.16 81) (end 167.5 78.66) (width 0.2) (layer "F.Cu") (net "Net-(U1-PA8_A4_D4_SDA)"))
 (segment (start 169.926346 82.59) (end 153.4 82.59) (width 0.2) (layer "F.Cu") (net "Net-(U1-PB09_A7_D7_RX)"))
 (segment (start 207.621 98.95247) (end 192.66853 84) (width 0.2) (layer "F.Cu") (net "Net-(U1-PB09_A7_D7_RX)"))
 (segment (start 171.336346 84) (end 169.926346 82.59) (width 0.2) (layer "F.Cu") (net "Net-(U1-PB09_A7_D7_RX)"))
 (segment (start 153.4 82.59) (end 152.25 83.74) (width 0.2) (layer "F.Cu") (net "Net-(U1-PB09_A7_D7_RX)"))
 (segment (start 192.66853 84) (end 171.336346 84) (width 0.2) (layer "F.Cu") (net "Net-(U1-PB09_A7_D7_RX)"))
 (segment (start 134.408831 100) (end 135.510101 101.10127) (width 0.2) (layer "F.Cu") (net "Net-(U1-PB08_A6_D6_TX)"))
 (segment (start 117 100) (end 134.408831 100) (width 0.2) (layer "F.Cu") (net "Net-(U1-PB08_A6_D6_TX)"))
 (segment (start 150.13873 101.10127) (end 167.5 83.74) (width 0.2) (layer "F.Cu") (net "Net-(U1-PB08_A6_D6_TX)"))
 (segment (start 135.510101 101.10127) (end 150.13873 101.10127) (width 0.2) (layer "F.Cu") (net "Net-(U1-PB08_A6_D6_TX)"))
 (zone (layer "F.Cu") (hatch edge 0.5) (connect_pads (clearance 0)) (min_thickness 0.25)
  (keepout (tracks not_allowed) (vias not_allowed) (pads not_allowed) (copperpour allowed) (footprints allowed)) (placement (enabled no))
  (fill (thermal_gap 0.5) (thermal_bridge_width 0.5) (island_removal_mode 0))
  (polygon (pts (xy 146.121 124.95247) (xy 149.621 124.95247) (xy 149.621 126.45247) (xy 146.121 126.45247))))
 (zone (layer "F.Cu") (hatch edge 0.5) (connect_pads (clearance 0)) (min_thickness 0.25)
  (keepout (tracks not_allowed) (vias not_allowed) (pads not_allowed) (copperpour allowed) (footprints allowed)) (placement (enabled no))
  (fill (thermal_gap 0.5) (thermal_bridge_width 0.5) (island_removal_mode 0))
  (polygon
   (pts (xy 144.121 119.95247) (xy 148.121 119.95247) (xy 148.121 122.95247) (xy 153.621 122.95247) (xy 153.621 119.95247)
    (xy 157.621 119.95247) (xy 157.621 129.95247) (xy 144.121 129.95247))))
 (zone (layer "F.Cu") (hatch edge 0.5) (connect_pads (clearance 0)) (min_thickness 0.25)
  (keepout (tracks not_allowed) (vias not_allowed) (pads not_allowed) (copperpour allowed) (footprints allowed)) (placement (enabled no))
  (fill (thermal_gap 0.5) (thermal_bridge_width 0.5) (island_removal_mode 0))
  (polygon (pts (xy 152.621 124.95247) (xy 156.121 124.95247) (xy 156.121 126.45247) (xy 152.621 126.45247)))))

